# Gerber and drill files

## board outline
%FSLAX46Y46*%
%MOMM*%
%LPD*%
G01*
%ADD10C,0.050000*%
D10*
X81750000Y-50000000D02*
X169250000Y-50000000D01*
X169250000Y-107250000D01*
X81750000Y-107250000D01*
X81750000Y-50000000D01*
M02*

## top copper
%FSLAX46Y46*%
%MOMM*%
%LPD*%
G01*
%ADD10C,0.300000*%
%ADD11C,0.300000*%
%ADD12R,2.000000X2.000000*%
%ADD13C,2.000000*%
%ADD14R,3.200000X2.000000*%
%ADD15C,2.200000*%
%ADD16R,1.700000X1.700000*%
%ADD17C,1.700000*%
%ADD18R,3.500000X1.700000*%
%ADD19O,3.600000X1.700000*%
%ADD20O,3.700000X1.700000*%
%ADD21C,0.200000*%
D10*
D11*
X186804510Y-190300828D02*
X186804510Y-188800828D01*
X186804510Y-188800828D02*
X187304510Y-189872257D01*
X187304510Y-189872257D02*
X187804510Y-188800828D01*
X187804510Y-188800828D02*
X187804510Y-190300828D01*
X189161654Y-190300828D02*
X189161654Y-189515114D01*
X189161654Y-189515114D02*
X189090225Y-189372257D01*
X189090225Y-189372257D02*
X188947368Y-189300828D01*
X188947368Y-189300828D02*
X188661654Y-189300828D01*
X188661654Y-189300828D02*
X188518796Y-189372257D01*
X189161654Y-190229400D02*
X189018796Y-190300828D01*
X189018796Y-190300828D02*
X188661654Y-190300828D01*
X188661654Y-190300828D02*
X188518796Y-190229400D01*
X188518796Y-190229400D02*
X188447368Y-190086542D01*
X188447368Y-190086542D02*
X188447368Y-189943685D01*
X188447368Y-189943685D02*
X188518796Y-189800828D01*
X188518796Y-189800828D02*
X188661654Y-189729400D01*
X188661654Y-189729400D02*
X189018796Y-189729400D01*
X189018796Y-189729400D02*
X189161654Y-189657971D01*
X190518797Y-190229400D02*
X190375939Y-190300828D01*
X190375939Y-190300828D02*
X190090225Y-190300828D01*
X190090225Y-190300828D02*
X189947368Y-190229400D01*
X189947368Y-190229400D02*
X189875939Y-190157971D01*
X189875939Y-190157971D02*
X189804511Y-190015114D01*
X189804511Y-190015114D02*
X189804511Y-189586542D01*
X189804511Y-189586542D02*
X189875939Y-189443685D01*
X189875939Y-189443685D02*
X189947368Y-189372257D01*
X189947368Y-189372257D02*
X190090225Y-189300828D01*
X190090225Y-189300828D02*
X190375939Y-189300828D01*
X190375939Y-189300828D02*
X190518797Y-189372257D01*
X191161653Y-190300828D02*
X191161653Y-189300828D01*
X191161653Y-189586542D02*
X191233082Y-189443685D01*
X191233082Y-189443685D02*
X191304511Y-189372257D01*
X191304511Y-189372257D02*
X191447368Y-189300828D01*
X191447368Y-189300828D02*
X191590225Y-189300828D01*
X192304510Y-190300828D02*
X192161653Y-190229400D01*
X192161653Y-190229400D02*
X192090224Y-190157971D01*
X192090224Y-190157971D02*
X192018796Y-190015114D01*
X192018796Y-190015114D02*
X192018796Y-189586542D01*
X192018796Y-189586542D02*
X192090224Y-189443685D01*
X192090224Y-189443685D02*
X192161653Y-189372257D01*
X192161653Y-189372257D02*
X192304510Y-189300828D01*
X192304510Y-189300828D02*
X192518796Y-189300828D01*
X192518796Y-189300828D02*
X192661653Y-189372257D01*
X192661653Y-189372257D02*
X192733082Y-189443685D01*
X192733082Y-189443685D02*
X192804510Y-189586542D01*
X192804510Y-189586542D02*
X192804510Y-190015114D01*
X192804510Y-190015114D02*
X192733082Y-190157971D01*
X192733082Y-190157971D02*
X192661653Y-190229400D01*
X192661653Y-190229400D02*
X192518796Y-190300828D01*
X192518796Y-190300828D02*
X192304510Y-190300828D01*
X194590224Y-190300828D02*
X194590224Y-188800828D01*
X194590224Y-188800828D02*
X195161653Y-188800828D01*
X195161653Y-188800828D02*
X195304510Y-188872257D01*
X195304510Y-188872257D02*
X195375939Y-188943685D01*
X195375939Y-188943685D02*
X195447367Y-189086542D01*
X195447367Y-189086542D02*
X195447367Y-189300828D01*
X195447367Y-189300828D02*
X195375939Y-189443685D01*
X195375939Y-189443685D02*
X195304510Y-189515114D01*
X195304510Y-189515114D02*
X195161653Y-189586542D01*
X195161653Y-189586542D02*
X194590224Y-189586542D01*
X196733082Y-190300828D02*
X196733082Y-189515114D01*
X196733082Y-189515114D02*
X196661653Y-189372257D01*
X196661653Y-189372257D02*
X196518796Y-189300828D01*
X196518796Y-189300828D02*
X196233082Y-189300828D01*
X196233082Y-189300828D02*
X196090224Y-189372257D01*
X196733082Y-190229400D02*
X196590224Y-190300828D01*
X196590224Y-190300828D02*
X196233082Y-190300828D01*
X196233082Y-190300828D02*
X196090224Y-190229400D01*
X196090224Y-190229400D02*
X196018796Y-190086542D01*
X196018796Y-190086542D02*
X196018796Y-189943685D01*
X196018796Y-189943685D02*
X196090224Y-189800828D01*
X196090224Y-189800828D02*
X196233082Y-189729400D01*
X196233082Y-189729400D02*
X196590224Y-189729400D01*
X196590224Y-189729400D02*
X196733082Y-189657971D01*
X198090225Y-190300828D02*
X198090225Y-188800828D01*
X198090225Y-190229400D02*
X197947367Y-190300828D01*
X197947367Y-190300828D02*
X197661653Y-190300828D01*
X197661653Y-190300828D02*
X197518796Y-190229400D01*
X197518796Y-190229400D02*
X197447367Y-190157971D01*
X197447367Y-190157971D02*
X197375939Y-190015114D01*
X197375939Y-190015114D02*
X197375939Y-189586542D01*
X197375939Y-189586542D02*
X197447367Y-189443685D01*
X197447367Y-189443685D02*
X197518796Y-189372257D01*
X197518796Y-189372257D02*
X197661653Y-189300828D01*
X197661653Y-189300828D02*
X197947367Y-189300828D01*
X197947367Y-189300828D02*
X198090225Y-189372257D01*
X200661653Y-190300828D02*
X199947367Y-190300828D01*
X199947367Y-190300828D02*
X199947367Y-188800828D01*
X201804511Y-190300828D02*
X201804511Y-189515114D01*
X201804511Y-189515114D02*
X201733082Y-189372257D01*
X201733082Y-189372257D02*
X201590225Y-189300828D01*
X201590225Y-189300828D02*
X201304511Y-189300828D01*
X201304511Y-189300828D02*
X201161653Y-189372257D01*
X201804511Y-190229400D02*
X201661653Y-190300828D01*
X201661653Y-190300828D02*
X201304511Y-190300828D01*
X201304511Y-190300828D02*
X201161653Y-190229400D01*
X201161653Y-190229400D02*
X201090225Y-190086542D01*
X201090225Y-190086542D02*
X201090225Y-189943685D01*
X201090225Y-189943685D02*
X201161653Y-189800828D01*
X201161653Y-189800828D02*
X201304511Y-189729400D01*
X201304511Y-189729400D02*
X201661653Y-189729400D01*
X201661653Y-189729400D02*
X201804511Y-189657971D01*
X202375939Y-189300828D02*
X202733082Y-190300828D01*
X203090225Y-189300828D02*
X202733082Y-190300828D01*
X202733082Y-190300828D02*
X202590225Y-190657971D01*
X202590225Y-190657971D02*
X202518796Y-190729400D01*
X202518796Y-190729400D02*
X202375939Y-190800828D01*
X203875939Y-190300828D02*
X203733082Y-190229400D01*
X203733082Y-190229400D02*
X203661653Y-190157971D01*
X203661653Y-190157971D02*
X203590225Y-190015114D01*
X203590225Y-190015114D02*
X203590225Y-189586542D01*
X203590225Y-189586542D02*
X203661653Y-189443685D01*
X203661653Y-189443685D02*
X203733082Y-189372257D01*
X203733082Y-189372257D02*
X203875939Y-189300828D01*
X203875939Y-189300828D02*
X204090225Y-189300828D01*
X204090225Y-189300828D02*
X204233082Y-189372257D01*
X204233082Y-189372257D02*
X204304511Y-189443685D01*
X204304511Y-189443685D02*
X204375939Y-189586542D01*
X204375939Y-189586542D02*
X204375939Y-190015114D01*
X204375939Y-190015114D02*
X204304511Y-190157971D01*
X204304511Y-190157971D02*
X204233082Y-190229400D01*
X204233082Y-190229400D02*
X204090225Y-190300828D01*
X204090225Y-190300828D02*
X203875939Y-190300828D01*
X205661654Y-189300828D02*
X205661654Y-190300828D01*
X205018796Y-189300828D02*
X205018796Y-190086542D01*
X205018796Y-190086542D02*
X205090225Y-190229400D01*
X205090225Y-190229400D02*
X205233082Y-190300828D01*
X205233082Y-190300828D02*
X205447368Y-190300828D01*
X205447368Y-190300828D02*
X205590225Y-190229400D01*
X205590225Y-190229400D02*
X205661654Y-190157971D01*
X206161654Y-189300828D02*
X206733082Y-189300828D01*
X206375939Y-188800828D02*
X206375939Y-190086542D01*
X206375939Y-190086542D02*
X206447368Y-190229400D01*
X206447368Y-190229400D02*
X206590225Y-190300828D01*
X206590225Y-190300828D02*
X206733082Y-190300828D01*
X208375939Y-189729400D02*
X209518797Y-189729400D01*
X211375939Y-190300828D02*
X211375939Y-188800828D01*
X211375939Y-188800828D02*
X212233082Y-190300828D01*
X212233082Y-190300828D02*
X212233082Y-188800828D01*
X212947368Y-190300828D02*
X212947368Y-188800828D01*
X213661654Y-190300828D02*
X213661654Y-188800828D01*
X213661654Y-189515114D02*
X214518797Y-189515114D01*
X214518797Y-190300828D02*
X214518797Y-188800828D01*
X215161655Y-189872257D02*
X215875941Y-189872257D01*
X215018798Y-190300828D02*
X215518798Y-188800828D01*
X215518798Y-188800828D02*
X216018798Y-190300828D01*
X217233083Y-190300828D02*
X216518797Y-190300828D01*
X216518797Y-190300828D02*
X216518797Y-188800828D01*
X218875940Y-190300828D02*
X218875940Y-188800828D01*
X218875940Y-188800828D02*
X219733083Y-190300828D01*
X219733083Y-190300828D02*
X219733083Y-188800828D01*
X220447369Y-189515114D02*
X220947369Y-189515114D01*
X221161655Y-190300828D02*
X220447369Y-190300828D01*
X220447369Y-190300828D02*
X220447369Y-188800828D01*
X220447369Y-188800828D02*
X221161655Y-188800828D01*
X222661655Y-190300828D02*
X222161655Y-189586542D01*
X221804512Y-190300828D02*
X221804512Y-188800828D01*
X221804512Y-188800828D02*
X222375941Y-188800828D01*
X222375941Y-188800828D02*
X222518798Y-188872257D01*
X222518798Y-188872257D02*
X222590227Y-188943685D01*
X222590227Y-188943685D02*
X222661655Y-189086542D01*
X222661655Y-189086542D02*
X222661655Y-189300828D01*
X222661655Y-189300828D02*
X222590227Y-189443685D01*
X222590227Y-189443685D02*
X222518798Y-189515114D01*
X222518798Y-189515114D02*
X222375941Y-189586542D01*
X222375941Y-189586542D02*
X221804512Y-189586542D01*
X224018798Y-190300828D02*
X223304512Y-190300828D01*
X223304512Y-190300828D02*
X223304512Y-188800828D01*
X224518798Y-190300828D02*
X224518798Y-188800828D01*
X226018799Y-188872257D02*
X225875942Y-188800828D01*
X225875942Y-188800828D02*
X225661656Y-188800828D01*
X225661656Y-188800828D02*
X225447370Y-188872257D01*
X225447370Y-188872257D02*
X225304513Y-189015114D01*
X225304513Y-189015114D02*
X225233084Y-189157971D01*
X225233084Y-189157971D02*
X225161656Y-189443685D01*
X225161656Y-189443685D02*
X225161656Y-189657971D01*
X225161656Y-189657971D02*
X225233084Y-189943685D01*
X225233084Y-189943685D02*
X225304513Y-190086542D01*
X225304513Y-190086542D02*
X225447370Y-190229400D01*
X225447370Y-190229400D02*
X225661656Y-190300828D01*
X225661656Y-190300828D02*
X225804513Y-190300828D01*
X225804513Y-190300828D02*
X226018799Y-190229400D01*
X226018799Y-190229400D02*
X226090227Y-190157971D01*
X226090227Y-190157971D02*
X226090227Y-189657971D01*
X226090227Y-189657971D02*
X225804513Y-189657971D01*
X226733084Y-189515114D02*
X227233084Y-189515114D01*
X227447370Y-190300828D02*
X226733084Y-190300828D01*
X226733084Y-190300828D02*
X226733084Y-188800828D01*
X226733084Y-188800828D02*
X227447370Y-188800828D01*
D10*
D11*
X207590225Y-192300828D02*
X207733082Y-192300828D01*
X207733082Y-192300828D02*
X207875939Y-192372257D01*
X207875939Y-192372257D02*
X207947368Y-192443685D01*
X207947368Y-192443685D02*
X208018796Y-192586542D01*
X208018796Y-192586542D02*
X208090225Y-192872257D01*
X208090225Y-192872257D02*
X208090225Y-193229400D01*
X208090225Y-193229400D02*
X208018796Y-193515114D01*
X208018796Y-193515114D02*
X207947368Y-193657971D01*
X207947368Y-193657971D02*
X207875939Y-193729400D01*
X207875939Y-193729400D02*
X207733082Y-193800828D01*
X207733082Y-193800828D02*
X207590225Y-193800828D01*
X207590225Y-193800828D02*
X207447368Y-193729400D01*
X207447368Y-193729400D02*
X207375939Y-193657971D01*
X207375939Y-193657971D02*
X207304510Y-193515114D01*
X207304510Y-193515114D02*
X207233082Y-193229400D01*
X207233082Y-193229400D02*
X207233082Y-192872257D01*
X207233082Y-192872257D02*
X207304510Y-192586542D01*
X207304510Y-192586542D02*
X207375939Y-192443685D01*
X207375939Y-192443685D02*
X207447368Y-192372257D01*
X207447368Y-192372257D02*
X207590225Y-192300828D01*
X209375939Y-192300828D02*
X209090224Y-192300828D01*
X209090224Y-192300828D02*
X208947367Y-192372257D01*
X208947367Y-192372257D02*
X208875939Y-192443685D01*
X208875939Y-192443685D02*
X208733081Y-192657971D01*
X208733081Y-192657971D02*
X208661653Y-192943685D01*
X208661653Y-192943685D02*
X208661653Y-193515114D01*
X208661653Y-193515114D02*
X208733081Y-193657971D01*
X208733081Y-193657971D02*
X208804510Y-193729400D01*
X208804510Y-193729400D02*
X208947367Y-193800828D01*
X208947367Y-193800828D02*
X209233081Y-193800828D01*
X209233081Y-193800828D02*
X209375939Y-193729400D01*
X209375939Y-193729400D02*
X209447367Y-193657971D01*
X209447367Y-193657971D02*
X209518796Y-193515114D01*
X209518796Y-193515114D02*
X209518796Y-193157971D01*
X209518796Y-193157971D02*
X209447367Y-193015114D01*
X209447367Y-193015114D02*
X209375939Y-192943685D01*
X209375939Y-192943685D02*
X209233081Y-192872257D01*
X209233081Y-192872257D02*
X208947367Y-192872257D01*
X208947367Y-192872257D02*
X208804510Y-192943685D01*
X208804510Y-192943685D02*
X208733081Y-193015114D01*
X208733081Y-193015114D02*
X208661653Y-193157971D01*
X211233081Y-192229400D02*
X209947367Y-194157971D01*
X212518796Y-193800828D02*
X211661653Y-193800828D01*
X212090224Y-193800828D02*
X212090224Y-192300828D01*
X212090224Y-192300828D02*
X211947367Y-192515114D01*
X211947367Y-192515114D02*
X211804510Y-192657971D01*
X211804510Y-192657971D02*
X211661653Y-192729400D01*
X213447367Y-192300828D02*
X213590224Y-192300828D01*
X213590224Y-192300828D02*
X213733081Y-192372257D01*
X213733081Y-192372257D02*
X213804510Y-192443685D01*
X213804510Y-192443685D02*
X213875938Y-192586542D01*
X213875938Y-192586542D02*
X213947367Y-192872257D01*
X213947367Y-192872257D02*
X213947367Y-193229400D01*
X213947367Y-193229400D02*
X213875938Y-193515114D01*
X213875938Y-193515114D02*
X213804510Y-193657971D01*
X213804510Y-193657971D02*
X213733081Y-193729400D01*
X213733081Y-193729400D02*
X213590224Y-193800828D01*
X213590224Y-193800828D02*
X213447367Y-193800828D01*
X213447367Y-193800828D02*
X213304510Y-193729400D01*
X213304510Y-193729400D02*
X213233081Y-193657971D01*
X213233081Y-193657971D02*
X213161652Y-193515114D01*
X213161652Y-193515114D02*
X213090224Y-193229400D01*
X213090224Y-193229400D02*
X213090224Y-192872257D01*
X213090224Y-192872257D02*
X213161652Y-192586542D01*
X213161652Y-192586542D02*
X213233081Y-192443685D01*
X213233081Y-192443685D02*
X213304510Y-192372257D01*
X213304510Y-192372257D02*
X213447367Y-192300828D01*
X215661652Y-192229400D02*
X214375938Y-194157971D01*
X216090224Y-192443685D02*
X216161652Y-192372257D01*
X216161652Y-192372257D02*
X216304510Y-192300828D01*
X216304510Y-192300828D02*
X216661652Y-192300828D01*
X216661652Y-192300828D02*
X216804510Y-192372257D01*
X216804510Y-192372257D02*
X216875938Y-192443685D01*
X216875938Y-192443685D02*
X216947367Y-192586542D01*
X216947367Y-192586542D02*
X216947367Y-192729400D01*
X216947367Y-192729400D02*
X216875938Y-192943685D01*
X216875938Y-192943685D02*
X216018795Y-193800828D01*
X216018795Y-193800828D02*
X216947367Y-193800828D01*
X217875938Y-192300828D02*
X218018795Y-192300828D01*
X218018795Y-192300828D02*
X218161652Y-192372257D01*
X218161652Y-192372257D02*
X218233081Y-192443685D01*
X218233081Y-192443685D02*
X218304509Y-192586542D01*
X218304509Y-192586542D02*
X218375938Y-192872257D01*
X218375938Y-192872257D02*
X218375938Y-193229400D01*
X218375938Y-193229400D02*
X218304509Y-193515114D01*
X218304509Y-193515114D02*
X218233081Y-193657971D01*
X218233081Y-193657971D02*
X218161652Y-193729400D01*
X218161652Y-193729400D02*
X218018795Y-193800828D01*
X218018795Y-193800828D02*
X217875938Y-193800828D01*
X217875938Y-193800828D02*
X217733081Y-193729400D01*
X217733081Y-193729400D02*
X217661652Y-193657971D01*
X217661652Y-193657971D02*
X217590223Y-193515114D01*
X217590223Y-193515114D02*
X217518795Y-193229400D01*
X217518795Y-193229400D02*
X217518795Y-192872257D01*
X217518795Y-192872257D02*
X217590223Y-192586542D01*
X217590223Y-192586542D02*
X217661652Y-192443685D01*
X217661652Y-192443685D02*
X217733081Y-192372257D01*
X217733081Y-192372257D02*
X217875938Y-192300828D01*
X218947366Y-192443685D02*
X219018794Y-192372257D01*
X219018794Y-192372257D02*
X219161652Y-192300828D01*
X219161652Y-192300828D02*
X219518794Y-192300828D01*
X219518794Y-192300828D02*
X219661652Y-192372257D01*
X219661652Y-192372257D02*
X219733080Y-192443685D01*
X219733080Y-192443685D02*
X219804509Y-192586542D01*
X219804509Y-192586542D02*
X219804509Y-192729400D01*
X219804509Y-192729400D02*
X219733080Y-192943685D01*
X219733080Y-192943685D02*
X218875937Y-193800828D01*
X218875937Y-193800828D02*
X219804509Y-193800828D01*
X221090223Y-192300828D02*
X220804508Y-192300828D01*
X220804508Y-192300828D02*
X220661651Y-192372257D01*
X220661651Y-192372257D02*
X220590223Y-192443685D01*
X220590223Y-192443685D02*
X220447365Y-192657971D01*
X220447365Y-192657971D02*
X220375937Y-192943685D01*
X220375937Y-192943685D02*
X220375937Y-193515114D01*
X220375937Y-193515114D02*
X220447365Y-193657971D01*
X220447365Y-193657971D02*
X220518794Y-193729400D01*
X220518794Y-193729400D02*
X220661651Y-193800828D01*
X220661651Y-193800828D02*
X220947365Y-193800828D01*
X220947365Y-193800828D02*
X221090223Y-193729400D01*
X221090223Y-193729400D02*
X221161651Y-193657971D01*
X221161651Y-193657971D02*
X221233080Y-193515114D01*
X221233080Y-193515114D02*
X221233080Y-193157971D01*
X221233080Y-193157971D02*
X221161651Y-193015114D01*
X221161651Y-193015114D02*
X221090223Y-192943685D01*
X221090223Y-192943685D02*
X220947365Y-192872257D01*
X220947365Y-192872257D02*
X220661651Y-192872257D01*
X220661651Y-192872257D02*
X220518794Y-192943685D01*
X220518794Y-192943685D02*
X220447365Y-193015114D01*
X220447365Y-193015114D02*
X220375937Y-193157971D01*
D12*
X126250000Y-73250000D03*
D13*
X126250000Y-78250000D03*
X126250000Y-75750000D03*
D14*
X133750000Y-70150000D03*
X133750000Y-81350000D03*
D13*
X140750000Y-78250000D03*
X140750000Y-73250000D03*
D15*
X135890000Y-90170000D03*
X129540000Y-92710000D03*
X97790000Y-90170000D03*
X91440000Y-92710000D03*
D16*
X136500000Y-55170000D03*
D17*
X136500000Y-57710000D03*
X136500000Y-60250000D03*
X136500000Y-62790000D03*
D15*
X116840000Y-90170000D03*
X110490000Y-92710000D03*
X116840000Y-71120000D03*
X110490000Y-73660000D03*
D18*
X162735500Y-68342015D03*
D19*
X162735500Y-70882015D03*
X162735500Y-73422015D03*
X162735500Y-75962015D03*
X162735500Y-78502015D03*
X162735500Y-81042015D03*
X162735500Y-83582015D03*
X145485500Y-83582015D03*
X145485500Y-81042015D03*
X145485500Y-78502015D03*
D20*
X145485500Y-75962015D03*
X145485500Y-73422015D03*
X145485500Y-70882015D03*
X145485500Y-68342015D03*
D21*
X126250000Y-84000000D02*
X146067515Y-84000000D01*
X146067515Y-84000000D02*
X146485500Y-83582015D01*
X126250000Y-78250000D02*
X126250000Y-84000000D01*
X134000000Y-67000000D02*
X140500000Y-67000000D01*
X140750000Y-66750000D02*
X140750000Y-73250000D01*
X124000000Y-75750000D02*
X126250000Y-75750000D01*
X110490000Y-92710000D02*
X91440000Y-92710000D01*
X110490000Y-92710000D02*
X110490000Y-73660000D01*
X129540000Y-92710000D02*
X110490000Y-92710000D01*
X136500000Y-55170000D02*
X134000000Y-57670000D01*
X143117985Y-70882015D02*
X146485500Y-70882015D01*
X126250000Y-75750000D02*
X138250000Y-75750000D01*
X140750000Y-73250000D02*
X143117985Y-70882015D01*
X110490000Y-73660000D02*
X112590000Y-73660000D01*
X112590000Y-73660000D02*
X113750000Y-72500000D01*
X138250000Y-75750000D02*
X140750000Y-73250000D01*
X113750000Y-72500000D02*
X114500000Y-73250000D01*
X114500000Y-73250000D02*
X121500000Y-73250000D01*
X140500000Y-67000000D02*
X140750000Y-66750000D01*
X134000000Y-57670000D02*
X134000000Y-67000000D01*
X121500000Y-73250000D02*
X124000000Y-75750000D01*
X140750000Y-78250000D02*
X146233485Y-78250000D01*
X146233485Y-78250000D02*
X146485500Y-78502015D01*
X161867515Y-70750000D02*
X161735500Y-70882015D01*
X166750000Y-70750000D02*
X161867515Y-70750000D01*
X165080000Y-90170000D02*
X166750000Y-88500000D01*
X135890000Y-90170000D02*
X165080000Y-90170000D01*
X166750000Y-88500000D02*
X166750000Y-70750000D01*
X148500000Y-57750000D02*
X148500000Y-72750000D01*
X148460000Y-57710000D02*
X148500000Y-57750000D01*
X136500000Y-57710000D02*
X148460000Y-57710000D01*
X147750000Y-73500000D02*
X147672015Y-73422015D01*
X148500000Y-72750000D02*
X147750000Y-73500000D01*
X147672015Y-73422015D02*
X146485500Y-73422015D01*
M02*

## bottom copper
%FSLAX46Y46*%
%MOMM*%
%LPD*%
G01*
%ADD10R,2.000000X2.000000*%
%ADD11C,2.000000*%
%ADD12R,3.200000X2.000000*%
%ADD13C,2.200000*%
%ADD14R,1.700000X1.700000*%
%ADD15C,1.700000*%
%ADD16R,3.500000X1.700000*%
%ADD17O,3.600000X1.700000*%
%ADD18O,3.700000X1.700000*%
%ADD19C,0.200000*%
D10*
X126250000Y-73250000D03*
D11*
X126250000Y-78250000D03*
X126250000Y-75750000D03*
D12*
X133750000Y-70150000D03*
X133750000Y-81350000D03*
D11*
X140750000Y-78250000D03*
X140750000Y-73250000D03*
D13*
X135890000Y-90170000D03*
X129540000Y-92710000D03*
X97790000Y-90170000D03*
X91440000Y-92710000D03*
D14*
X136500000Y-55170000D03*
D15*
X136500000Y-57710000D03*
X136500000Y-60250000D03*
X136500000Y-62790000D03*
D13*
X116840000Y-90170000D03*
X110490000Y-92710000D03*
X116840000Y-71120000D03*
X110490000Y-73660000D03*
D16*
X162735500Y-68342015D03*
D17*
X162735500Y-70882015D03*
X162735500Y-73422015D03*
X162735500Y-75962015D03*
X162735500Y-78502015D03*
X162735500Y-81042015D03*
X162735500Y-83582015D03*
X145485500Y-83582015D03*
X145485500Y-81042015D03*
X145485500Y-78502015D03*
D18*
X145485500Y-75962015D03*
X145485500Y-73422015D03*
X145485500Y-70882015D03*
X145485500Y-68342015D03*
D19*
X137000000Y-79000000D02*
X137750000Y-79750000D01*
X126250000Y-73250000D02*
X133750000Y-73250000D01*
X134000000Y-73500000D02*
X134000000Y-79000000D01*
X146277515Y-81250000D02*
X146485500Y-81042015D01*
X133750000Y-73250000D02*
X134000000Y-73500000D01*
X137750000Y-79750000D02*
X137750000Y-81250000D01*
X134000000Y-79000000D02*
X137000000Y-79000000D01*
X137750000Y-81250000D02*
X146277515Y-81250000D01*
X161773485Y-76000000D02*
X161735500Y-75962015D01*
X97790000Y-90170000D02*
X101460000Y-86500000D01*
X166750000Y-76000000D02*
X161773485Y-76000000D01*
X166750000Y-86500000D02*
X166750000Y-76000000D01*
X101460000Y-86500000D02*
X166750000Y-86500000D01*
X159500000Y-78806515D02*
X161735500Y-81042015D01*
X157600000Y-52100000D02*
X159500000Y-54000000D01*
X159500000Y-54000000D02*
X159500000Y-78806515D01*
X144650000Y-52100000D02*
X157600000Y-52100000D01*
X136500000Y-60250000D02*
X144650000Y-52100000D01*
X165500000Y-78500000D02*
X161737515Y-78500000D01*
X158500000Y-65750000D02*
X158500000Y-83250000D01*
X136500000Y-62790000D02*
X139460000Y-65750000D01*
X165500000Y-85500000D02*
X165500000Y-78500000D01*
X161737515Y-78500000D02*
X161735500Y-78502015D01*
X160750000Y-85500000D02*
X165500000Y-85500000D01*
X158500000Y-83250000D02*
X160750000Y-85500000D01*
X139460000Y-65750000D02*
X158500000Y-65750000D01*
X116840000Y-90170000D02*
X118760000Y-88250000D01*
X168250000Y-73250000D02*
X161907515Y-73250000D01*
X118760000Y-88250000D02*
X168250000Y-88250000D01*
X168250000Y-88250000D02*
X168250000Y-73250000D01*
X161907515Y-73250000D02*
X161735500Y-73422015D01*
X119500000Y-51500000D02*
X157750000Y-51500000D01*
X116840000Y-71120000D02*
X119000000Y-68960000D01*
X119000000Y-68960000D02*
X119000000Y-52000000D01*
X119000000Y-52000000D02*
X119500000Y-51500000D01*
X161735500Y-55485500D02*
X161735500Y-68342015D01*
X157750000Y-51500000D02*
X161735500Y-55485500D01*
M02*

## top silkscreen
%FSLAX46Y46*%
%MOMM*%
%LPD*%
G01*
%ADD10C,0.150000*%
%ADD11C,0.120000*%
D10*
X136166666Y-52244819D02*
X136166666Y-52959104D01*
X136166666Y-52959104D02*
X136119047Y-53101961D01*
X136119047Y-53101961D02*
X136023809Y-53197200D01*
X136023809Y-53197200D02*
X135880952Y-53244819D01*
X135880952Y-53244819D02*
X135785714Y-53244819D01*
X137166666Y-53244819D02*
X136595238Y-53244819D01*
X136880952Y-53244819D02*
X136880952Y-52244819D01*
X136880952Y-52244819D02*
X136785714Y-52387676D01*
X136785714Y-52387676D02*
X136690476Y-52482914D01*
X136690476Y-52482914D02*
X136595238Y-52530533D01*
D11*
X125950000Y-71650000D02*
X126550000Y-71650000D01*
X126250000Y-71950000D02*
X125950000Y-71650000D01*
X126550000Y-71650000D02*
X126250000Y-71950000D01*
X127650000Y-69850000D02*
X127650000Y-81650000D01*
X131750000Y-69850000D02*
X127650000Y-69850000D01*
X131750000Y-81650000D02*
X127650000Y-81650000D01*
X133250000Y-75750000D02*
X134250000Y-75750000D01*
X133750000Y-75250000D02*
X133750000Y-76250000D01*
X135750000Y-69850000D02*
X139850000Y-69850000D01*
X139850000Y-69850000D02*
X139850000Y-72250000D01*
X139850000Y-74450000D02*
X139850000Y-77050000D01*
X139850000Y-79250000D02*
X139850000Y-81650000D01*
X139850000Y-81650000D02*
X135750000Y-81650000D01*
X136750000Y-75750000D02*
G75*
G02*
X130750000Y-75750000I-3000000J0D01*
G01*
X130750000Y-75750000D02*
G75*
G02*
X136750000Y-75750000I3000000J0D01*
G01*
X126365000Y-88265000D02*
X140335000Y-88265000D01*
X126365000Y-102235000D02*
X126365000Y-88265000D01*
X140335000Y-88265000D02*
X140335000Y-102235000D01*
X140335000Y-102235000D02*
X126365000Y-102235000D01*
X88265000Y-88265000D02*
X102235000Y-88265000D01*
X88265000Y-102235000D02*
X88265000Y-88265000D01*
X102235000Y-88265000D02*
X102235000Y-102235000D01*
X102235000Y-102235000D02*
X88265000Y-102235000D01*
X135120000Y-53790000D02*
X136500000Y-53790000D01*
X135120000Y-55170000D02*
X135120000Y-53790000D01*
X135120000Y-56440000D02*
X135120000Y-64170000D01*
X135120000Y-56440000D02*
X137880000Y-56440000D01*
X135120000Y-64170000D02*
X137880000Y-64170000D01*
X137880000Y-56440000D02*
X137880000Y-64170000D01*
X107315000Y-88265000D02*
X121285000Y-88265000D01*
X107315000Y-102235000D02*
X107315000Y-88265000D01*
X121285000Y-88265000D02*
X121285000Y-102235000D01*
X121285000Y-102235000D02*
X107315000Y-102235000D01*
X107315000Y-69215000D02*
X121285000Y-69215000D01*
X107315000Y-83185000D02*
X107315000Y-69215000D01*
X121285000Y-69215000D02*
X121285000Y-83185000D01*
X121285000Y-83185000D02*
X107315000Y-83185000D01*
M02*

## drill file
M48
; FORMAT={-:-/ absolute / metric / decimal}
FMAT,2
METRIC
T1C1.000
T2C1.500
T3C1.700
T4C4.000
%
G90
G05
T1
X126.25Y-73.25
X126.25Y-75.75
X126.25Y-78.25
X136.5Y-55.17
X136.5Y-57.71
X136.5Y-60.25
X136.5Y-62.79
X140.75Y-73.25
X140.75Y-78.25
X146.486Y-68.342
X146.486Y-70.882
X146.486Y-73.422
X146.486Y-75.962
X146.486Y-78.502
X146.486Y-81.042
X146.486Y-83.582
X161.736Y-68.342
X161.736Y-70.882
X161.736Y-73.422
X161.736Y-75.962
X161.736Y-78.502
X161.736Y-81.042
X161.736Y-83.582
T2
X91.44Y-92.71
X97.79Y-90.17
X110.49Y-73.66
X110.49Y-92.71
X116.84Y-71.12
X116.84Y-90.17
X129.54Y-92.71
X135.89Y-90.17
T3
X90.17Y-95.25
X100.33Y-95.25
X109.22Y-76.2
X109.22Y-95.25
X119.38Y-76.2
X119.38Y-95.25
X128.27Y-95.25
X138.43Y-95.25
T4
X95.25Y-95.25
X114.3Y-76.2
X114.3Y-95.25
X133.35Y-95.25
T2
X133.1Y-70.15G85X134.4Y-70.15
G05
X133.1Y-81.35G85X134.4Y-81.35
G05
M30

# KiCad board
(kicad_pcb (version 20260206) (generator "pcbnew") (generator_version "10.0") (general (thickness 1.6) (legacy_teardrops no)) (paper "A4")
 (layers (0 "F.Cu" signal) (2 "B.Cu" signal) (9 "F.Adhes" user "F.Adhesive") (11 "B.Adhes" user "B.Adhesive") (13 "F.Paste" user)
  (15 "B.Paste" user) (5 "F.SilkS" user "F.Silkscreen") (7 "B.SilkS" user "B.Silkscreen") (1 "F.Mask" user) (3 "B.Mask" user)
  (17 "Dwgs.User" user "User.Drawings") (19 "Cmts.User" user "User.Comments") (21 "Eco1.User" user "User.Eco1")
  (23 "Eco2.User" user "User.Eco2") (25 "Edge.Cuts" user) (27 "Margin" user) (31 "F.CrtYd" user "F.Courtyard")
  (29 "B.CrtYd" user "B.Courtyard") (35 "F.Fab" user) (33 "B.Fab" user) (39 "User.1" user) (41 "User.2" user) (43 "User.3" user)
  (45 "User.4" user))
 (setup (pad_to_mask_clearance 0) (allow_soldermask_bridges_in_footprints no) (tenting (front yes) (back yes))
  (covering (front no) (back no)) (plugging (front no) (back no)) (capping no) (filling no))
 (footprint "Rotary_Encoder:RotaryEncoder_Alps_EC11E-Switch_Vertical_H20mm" (layer "F.Cu") (at 126.25 73.25)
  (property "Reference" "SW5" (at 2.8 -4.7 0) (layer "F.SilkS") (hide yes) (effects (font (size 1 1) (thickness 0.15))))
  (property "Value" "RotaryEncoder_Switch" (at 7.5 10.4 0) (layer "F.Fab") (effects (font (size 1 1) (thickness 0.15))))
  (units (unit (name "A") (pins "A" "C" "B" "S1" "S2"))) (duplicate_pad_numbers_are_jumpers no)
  (fp_line (start -0.3 -1.6) (end 0.3 -1.6) (stroke (width 0.12) (type solid)) (layer "F.SilkS"))
  (fp_line (start 0 -1.3) (end -0.3 -1.6) (stroke (width 0.12) (type solid)) (layer "F.SilkS"))
  (fp_line (start 0.3 -1.6) (end 0 -1.3) (stroke (width 0.12) (type solid)) (layer "F.SilkS"))
  (fp_line (start 1.4 -3.4) (end 1.4 8.4) (stroke (width 0.12) (type solid)) (layer "F.SilkS"))
  (fp_line (start 5.5 -3.4) (end 1.4 -3.4) (stroke (width 0.12) (type solid)) (layer "F.SilkS"))
  (fp_line (start 5.5 8.4) (end 1.4 8.4) (stroke (width 0.12) (type solid)) (layer "F.SilkS"))
  (fp_line (start 7 2.5) (end 8 2.5) (stroke (width 0.12) (type solid)) (layer "F.SilkS"))
  (fp_line (start 7.5 2) (end 7.5 3) (stroke (width 0.12) (type solid)) (layer "F.SilkS"))
  (fp_line (start 9.5 -3.4) (end 13.6 -3.4) (stroke (width 0.12) (type solid)) (layer "F.SilkS"))
  (fp_line (start 13.6 -3.4) (end 13.6 -1) (stroke (width 0.12) (type solid)) (layer "F.SilkS"))
  (fp_line (start 13.6 1.2) (end 13.6 3.8) (stroke (width 0.12) (type solid)) (layer "F.SilkS"))
  (fp_line (start 13.6 6) (end 13.6 8.4) (stroke (width 0.12) (type solid)) (layer "F.SilkS"))
  (fp_line (start 13.6 8.4) (end 9.5 8.4) (stroke (width 0.12) (type solid)) (layer "F.SilkS"))
  (fp_circle (center 7.5 2.5) (end 10.5 2.5) (stroke (width 0.12) (type solid)) (fill no) (layer "F.SilkS"))
  (pad "A" thru_hole rect (at 0 0) (size 2 2) (drill 1) (layers "*.Cu" "*.Mask") (remove_unused_layers no) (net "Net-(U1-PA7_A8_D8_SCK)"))
  (pad "B" thru_hole circle (at 0 5) (size 2 2) (drill 1) (layers "*.Cu" "*.Mask") (remove_unused_layers no) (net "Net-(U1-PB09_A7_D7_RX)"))
  (pad "C" thru_hole circle (at 0 2.5) (size 2 2) (drill 1) (layers "*.Cu" "*.Mask") (remove_unused_layers no) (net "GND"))
  (pad "MP" thru_hole rect (at 7.5 -3.1) (size 3.2 2) (drill oval 2.8 1.5) (layers "*.Cu" "*.Mask") (remove_unused_layers no))
  (pad "MP" thru_hole rect (at 7.5 8.1) (size 3.2 2) (drill oval 2.8 1.5) (layers "*.Cu" "*.Mask") (remove_unused_layers no))
  (pad "S1" thru_hole circle (at 14.5 5) (size 2 2) (drill 1) (layers "*.Cu" "*.Mask") (remove_unused_layers no)
   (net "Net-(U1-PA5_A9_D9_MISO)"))
  (pad "S2" thru_hole circle (at 14.5 0) (size 2 2) (drill 1) (layers "*.Cu" "*.Mask") (remove_unused_layers no) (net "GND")))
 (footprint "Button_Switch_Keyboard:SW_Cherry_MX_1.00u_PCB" (layer "F.Cu") (at 135.89 90.17)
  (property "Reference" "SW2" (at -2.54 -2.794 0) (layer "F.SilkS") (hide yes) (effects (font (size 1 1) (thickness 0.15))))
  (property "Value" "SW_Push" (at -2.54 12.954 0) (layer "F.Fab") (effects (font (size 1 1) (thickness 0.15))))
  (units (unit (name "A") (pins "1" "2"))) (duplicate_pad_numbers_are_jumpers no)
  (fp_line (start -9.525 -1.905) (end 4.445 -1.905) (stroke (width 0.12) (type solid)) (layer "F.SilkS"))
  (fp_line (start -9.525 12.065) (end -9.525 -1.905) (stroke (width 0.12) (type solid)) (layer "F.SilkS"))
  (fp_line (start 4.445 -1.905) (end 4.445 12.065) (stroke (width 0.12) (type solid)) (layer "F.SilkS"))
  (fp_line (start 4.445 12.065) (end -9.525 12.065) (stroke (width 0.12) (type solid)) (layer "F.SilkS"))
  (pad "" np_thru_hole circle (at -7.62 5.08) (size 1.7 1.7) (drill 1.7) (layers "*.Cu" "*.Mask"))
  (pad "" np_thru_hole circle (at -2.54 5.08) (size 4 4) (drill 4) (layers "*.Cu" "*.Mask"))
  (pad "" np_thru_hole circle (at 2.54 5.08) (size 1.7 1.7) (drill 1.7) (layers "*.Cu" "*.Mask"))
  (pad "1" thru_hole circle (at 0 0) (size 2.2 2.2) (drill 1.5) (layers "*.Cu" "*.Mask") (remove_unused_layers no)
   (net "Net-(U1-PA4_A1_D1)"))
  (pad "2" thru_hole circle (at -6.35 2.54) (size 2.2 2.2) (drill 1.5) (layers "*.Cu" "*.Mask") (remove_unused_layers no) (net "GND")))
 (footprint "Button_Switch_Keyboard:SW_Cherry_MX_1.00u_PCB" (layer "F.Cu") (at 97.79 90.17)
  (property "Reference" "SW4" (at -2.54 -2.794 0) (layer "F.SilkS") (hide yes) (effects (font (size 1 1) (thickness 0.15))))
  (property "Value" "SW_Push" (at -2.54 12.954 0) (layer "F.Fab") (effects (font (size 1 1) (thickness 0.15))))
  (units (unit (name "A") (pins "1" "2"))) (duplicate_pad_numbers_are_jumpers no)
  (fp_line (start -9.525 -1.905) (end 4.445 -1.905) (stroke (width 0.12) (type solid)) (layer "F.SilkS"))
  (fp_line (start -9.525 12.065) (end -9.525 -1.905) (stroke (width 0.12) (type solid)) (layer "F.SilkS"))
  (fp_line (start 4.445 -1.905) (end 4.445 12.065) (stroke (width 0.12) (type solid)) (layer "F.SilkS"))
  (fp_line (start 4.445 12.065) (end -9.525 12.065) (stroke (width 0.12) (type solid)) (layer "F.SilkS"))
  (pad "" np_thru_hole circle (at -7.62 5.08) (size 1.7 1.7) (drill 1.7) (layers "*.Cu" "*.Mask"))
  (pad "" np_thru_hole circle (at -2.54 5.08) (size 4 4) (drill 4) (layers "*.Cu" "*.Mask"))
  (pad "" np_thru_hole circle (at 2.54 5.08) (size 1.7 1.7) (drill 1.7) (layers "*.Cu" "*.Mask"))
  (pad "1" thru_hole circle (at 0 0) (size 2.2 2.2) (drill 1.5) (layers "*.Cu" "*.Mask") (remove_unused_layers no)
   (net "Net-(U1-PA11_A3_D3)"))
  (pad "2" thru_hole circle (at -6.35 2.54) (size 2.2 2.2) (drill 1.5) (layers "*.Cu" "*.Mask") (remove_unused_layers no) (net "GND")))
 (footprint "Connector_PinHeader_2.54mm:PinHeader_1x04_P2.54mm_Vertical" (layer "F.Cu") (at 136.5 55.17)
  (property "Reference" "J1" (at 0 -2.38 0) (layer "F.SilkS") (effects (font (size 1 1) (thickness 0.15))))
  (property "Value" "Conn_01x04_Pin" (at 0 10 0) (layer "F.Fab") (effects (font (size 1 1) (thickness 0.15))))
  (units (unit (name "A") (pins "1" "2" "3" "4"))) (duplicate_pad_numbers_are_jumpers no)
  (fp_line (start -1.38 -1.38) (end 0 -1.38) (stroke (width 0.12) (type solid)) (layer "F.SilkS"))
  (fp_line (start -1.38 0) (end -1.38 -1.38) (stroke (width 0.12) (type solid)) (layer "F.SilkS"))
  (fp_line (start -1.38 1.27) (end -1.38 9) (stroke (width 0.12) (type solid)) (layer "F.SilkS"))
  (fp_line (start -1.38 1.27) (end 1.38 1.27) (stroke (width 0.12) (type solid)) (layer "F.SilkS"))
  (fp_line (start -1.38 9) (end 1.38 9) (stroke (width 0.12) (type solid)) (layer "F.SilkS"))
  (fp_line (start 1.38 1.27) (end 1.38 9) (stroke (width 0.12) (type solid)) (layer "F.SilkS"))
  (pad "1" thru_hole rect (at 0 0) (size 1.7 1.7) (drill 1) (layers "*.Cu" "*.Mask") (remove_unused_layers no) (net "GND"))
  (pad "2" thru_hole circle (at 0 2.54) (size 1.7 1.7) (drill 1) (layers "*.Cu" "*.Mask") (remove_unused_layers no) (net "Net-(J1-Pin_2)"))
  (pad "3" thru_hole circle (at 0 5.08) (size 1.7 1.7) (drill 1) (layers "*.Cu" "*.Mask") (remove_unused_layers no) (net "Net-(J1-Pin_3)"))
  (pad "4" thru_hole circle (at 0 7.62) (size 1.7 1.7) (drill 1) (layers "*.Cu" "*.Mask") (remove_unused_layers no) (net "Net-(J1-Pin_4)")))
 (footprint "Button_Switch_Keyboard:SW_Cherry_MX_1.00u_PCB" (layer "F.Cu") (at 116.84 90.17)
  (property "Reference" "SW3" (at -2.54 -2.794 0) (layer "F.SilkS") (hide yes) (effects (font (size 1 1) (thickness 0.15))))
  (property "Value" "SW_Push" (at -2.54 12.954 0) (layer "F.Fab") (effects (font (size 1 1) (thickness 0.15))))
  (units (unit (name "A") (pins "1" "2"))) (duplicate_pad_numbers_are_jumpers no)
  (fp_line (start -9.525 -1.905) (end 4.445 -1.905) (stroke (width 0.12) (type solid)) (layer "F.SilkS"))
  (fp_line (start -9.525 12.065) (end -9.525 -1.905) (stroke (width 0.12) (type solid)) (layer "F.SilkS"))
  (fp_line (start 4.445 -1.905) (end 4.445 12.065) (stroke (width 0.12) (type solid)) (layer "F.SilkS"))
  (fp_line (start 4.445 12.065) (end -9.525 12.065) (stroke (width 0.12) (type solid)) (layer "F.SilkS"))
  (pad "" np_thru_hole circle (at -7.62 5.08) (size 1.7 1.7) (drill 1.7) (layers "*.Cu" "*.Mask"))
  (pad "" np_thru_hole circle (at -2.54 5.08) (size 4 4) (drill 4) (layers "*.Cu" "*.Mask"))
  (pad "" np_thru_hole circle (at 2.54 5.08) (size 1.7 1.7) (drill 1.7) (layers "*.Cu" "*.Mask"))
  (pad "1" thru_hole circle (at 0 0) (size 2.2 2.2) (drill 1.5) (layers "*.Cu" "*.Mask") (remove_unused_layers no)
   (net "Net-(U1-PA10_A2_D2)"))
  (pad "2" thru_hole circle (at -6.35 2.54) (size 2.2 2.2) (drill 1.5) (layers "*.Cu" "*.Mask") (remove_unused_layers no) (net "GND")))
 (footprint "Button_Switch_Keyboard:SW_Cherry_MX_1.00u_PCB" (layer "F.Cu") (at 116.84 71.12)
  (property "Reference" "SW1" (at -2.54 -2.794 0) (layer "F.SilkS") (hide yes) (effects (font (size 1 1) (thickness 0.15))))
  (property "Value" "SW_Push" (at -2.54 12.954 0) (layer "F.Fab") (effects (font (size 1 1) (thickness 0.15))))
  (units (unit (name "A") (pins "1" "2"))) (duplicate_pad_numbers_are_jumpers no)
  (fp_line (start -9.525 -1.905) (end 4.445 -1.905) (stroke (width 0.12) (type solid)) (layer "F.SilkS"))
  (fp_line (start -9.525 12.065) (end -9.525 -1.905) (stroke (width 0.12) (type solid)) (layer "F.SilkS"))
  (fp_line (start 4.445 -1.905) (end 4.445 12.065) (stroke (width 0.12) (type solid)) (layer "F.SilkS"))
  (fp_line (start 4.445 12.065) (end -9.525 12.065) (stroke (width 0.12) (type solid)) (layer "F.SilkS"))
  (pad "" np_thru_hole circle (at -7.62 5.08) (size 1.7 1.7) (drill 1.7) (layers "*.Cu" "*.Mask"))
  (pad "" np_thru_hole circle (at -2.54 5.08) (size 4 4) (drill 4) (layers "*.Cu" "*.Mask"))
  (pad "" np_thru_hole circle (at 2.54 5.08) (size 1.7 1.7) (drill 1.7) (layers "*.Cu" "*.Mask"))
  (pad "1" thru_hole circle (at 0 0) (size 2.2 2.2) (drill 1.5) (layers "*.Cu" "*.Mask") (remove_unused_layers no)
   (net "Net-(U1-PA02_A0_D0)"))
  (pad "2" thru_hole circle (at -6.35 2.54) (size 2.2 2.2) (drill 1.5) (layers "*.Cu" "*.Mask") (remove_unused_layers no) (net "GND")))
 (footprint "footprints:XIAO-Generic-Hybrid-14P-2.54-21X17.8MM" (layer "B.Cu") (at 154.1105 75.962015 180)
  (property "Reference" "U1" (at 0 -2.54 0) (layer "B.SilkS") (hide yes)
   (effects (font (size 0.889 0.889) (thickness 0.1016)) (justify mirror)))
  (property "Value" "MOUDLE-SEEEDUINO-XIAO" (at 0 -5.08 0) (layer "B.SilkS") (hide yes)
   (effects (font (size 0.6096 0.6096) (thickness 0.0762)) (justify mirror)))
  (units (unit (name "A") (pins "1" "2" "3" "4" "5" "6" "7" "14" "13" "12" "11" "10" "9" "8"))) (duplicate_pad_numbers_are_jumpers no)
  (pad "1" thru_hole rect (at -7.625 7.62 180) (size 3.5 1.7) (drill 1 (offset -1 0)) (layers "*.Cu" "*.Mask") (remove_unused_layers no)
   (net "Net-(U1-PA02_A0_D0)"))
  (pad "2" thru_hole oval (at -7.625 5.08 180) (size 3.6 1.7) (drill 1 (offset -1 0)) (layers "*.Cu" "*.Mask") (remove_unused_layers no)
   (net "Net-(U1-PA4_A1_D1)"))
  (pad "3" thru_hole oval (at -7.625 2.54 180) (size 3.6 1.7) (drill 1 (offset -1 0)) (layers "*.Cu" "*.Mask") (remove_unused_layers no)
   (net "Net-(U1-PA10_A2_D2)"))
  (pad "4" thru_hole oval (at -7.625 0 180) (size 3.6 1.7) (drill 1 (offset -1 0)) (layers "*.Cu" "*.Mask") (remove_unused_layers no)
   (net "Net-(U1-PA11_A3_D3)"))
  (pad "5" thru_hole oval (at -7.625 -2.54 180) (size 3.6 1.7) (drill 1 (offset -1 0)) (layers "*.Cu" "*.Mask") (remove_unused_layers no)
   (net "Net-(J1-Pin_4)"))
  (pad "6" thru_hole oval (at -7.625 -5.08) (size 3.6 1.7) (drill 1 (offset 1 0)) (layers "*.Cu" "*.Mask") (remove_unused_layers no)
   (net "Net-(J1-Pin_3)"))
  (pad "7" thru_hole oval (at -7.625 -7.62 180) (size 3.6 1.7) (drill 1 (offset -1 0)) (layers "*.Cu" "*.Mask") (remove_unused_layers no)
   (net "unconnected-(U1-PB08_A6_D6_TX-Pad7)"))
  (pad "8" thru_hole oval (at 7.625 -7.62 180) (size 3.6 1.7) (drill 1 (offset 1 0)) (layers "*.Cu" "*.Mask") (remove_unused_layers no)
   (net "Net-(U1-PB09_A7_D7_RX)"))
  (pad "9" thru_hole oval (at 7.625 -5.08 180) (size 3.6 1.7) (drill 1 (offset 1 0)) (layers "*.Cu" "*.Mask") (remove_unused_layers no)
   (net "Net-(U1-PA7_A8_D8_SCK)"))
  (pad "10" thru_hole oval (at 7.625 -2.54 180) (size 3.6 1.7) (drill 1 (offset 1 0)) (layers "*.Cu" "*.Mask") (remove_unused_layers no)
   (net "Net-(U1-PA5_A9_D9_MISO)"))
  (pad "11" thru_hole oval (at 7.625 0 180) (size 3.7 1.7) (drill 1 (offset 1 0)) (layers "*.Cu" "*.Mask") (remove_unused_layers no)
   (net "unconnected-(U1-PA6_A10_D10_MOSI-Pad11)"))
  (pad "12" thru_hole oval (at 7.625 2.54 180) (size 3.7 1.7) (drill 1 (offset 1 0)) (layers "*.Cu" "*.Mask") (remove_unused_layers no)
   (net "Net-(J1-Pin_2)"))
  (pad "13" thru_hole oval (at 7.625 5.08 180) (size 3.7 1.7) (drill 1 (offset 1 0)) (layers "*.Cu" "*.Mask") (remove_unused_layers no)
   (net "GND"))
  (pad "14" thru_hole oval (at 7.625 7.62 180) (size 3.7 1.7) (drill 1 (offset 1 0)) (layers "*.Cu" "*.Mask") (remove_unused_layers no)
   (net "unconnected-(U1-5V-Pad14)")))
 (gr_rect (start 81.75 50) (end 169.25 107.25) (stroke (width 0.05) (type default)) (fill no) (layer "Edge.Cuts"))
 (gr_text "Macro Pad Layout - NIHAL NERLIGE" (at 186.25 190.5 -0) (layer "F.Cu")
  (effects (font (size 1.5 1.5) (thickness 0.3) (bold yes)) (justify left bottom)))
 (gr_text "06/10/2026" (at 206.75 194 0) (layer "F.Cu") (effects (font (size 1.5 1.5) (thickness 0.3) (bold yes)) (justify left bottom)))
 (segment (start 137 79) (end 137.75 79.75) (width 0.2) (layer "B.Cu") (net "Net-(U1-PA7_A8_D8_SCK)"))
 (segment (start 126.25 73.25) (end 133.75 73.25) (width 0.2) (layer "B.Cu") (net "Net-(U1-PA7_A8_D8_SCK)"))
 (segment (start 134 73.5) (end 134 79) (width 0.2) (layer "B.Cu") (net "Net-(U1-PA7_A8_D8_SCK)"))
 (segment (start 146.277515 81.25) (end 146.4855 81.042015) (width 0.2) (layer "B.Cu") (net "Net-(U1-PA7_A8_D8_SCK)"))
 (segment (start 133.75 73.25) (end 134 73.5) (width 0.2) (layer "B.Cu") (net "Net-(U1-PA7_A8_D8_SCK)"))
 (segment (start 137.75 79.75) (end 137.75 81.25) (width 0.2) (layer "B.Cu") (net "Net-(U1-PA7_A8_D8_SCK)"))
 (segment (start 134 79) (end 137 79) (width 0.2) (layer "B.Cu") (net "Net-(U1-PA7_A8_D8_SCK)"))
 (segment (start 137.75 81.25) (end 146.277515 81.25) (width 0.2) (layer "B.Cu") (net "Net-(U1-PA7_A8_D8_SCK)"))
 (segment (start 126.25 84) (end 146.067515 84) (width 0.2) (layer "F.Cu") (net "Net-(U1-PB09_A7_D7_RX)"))
 (segment (start 146.067515 84) (end 146.4855 83.582015) (width 0.2) (layer "F.Cu") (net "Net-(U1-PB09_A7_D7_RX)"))
 (segment (start 126.25 78.25) (end 126.25 84) (width 0.2) (layer "F.Cu") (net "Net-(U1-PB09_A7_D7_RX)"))
 (segment (start 134 67) (end 140.5 67) (width 0.2) (layer "F.Cu") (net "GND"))
 (segment (start 140.75 66.75) (end 140.75 73.25) (width 0.2) (layer "F.Cu") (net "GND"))
 (segment (start 124 75.75) (end 126.25 75.75) (width 0.2) (layer "F.Cu") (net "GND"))
 (segment (start 110.49 92.71) (end 91.44 92.71) (width 0.2) (layer "F.Cu") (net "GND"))
 (segment (start 110.49 92.71) (end 110.49 73.66) (width 0.2) (layer "F.Cu") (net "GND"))
 (segment (start 129.54 92.71) (end 110.49 92.71) (width 0.2) (layer "F.Cu") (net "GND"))
 (segment (start 136.5 55.17) (end 134 57.67) (width 0.2) (layer "F.Cu") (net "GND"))
 (segment (start 143.117985 70.882015) (end 146.4855 70.882015) (width 0.2) (layer "F.Cu") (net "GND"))
 (segment (start 126.25 75.75) (end 138.25 75.75) (width 0.2) (layer "F.Cu") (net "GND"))
 (segment (start 140.75 73.25) (end 143.117985 70.882015) (width 0.2) (layer "F.Cu") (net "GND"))
 (segment (start 110.49 73.66) (end 112.59 73.66) (width 0.2) (layer "F.Cu") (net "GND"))
 (segment (start 112.59 73.66) (end 113.75 72.5) (width 0.2) (layer "F.Cu") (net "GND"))
 (segment (start 138.25 75.75) (end 140.75 73.25) (width 0.2) (layer "F.Cu") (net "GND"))
 (segment (start 113.75 72.5) (end 114.5 73.25) (width 0.2) (layer "F.Cu") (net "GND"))
 (segment (start 114.5 73.25) (end 121.5 73.25) (width 0.2) (layer "F.Cu") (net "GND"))
 (segment (start 140.5 67) (end 140.75 66.75) (width 0.2) (layer "F.Cu") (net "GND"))
 (segment (start 134 57.67) (end 134 67) (width 0.2) (layer "F.Cu") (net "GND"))
 (segment (start 121.5 73.25) (end 124 75.75) (width 0.2) (layer "F.Cu") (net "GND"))
 (segment (start 140.75 78.25) (end 146.233485 78.25) (width 0.2) (layer "F.Cu") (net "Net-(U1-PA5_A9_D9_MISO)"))
 (segment (start 146.233485 78.25) (end 146.4855 78.502015) (width 0.2) (layer "F.Cu") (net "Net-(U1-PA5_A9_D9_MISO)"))
 (segment (start 161.867515 70.75) (end 161.7355 70.882015) (width 0.2) (layer "F.Cu") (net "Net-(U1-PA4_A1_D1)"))
 (segment (start 166.75 70.75) (end 161.867515 70.75) (width 0.2) (layer "F.Cu") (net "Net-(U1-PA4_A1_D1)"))
 (segment (start 165.08 90.17) (end 166.75 88.5) (width 0.2) (layer "F.Cu") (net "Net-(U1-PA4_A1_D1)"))
 (segment (start 135.89 90.17) (end 165.08 90.17) (width 0.2) (layer "F.Cu") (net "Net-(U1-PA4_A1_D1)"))
 (segment (start 166.75 88.5) (end 166.75 70.75) (width 0.2) (layer "F.Cu") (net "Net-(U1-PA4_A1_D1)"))
 (segment (start 161.773485 76) (end 161.7355 75.962015) (width 0.2) (layer "B.Cu") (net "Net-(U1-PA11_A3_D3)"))
 (segment (start 97.79 90.17) (end 101.46 86.5) (width 0.2) (layer "B.Cu") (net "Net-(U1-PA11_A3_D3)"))
 (segment (start 166.75 76) (end 161.773485 76) (width 0.2) (layer "B.Cu") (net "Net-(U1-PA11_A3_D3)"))
 (segment (start 166.75 86.5) (end 166.75 76) (width 0.2) (layer "B.Cu") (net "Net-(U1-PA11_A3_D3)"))
 (segment (start 101.46 86.5) (end 166.75 86.5) (width 0.2) (layer "B.Cu") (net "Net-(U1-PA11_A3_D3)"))
 (segment (start 148.5 57.75) (end 148.5 72.75) (width 0.2) (layer "F.Cu") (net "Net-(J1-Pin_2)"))
 (segment (start 148.46 57.71) (end 148.5 57.75) (width 0.2) (layer "F.Cu") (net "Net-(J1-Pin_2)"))
 (segment (start 136.5 57.71) (end 148.46 57.71) (width 0.2) (layer "F.Cu") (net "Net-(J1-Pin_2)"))
 (segment (start 147.75 73.5) (end 147.672015 73.422015) (width 0.2) (layer "F.Cu") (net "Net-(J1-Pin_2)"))
 (segment (start 148.5 72.75) (end 147.75 73.5) (width 0.2) (layer "F.Cu") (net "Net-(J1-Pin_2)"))
 (segment (start 147.672015 73.422015) (end 146.4855 73.422015) (width 0.2) (layer "F.Cu") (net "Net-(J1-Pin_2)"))
 (segment (start 159.5 78.806515) (end 161.7355 81.042015) (width 0.2) (layer "B.Cu") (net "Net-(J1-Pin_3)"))
 (segment (start 157.6 52.1) (end 159.5 54) (width 0.2) (layer "B.Cu") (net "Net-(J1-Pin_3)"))
 (segment (start 159.5 54) (end 159.5 78.806515) (width 0.2) (layer "B.Cu") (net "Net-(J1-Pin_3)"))
 (segment (start 144.65 52.1) (end 157.6 52.1) (width 0.2) (layer "B.Cu") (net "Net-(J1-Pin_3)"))
 (segment (start 136.5 60.25) (end 144.65 52.1) (width 0.2) (layer "B.Cu") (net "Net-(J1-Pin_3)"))
 (segment (start 165.5 78.5) (end 161.737515 78.5) (width 0.2) (layer "B.Cu") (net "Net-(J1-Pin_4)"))
 (segment (start 158.5 65.75) (end 158.5 83.25) (width 0.2) (layer "B.Cu") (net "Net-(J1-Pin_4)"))
 (segment (start 136.5 62.79) (end 139.46 65.75) (width 0.2) (layer "B.Cu") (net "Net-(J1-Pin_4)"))
 (segment (start 165.5 85.5) (end 165.5 78.5) (width 0.2) (layer "B.Cu") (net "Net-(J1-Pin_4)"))
 (segment (start 161.737515 78.5) (end 161.7355 78.502015) (width 0.2) (layer "B.Cu") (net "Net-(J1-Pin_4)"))
 (segment (start 160.75 85.5) (end 165.5 85.5) (width 0.2) (layer "B.Cu") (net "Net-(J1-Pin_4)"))
 (segment (start 158.5 83.25) (end 160.75 85.5) (width 0.2) (layer "B.Cu") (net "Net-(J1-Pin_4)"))
 (segment (start 139.46 65.75) (end 158.5 65.75) (width 0.2) (layer "B.Cu") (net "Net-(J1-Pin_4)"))
 (segment (start 116.84 90.17) (end 118.76 88.25) (width 0.2) (layer "B.Cu") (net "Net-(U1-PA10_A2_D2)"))
 (segment (start 168.25 73.25) (end 161.907515 73.25) (width 0.2) (layer "B.Cu") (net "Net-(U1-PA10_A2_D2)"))
 (segment (start 118.76 88.25) (end 168.25 88.25) (width 0.2) (layer "B.Cu") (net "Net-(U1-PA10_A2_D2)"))
 (segment (start 168.25 88.25) (end 168.25 73.25) (width 0.2) (layer "B.Cu") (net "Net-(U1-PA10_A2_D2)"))
 (segment (start 161.907515 73.25) (end 161.7355 73.422015) (width 0.2) (layer "B.Cu") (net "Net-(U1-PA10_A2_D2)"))
 (segment (start 119.5 51.5) (end 157.75 51.5) (width 0.2) (layer "B.Cu") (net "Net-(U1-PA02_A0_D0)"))
 (segment (start 116.84 71.12) (end 119 68.96) (width 0.2) (layer "B.Cu") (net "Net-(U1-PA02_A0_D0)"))
 (segment (start 119 68.96) (end 119 52) (width 0.2) (layer "B.Cu") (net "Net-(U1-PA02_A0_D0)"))
 (segment (start 119 52) (end 119.5 51.5) (width 0.2) (layer "B.Cu") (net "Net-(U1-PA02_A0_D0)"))
 (segment (start 161.7355 55.4855) (end 161.7355 68.342015) (width 0.2) (layer "B.Cu") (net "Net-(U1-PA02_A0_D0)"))
 (segment (start 157.75 51.5) (end 161.7355 55.4855) (width 0.2) (layer "B.Cu") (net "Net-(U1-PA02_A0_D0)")))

